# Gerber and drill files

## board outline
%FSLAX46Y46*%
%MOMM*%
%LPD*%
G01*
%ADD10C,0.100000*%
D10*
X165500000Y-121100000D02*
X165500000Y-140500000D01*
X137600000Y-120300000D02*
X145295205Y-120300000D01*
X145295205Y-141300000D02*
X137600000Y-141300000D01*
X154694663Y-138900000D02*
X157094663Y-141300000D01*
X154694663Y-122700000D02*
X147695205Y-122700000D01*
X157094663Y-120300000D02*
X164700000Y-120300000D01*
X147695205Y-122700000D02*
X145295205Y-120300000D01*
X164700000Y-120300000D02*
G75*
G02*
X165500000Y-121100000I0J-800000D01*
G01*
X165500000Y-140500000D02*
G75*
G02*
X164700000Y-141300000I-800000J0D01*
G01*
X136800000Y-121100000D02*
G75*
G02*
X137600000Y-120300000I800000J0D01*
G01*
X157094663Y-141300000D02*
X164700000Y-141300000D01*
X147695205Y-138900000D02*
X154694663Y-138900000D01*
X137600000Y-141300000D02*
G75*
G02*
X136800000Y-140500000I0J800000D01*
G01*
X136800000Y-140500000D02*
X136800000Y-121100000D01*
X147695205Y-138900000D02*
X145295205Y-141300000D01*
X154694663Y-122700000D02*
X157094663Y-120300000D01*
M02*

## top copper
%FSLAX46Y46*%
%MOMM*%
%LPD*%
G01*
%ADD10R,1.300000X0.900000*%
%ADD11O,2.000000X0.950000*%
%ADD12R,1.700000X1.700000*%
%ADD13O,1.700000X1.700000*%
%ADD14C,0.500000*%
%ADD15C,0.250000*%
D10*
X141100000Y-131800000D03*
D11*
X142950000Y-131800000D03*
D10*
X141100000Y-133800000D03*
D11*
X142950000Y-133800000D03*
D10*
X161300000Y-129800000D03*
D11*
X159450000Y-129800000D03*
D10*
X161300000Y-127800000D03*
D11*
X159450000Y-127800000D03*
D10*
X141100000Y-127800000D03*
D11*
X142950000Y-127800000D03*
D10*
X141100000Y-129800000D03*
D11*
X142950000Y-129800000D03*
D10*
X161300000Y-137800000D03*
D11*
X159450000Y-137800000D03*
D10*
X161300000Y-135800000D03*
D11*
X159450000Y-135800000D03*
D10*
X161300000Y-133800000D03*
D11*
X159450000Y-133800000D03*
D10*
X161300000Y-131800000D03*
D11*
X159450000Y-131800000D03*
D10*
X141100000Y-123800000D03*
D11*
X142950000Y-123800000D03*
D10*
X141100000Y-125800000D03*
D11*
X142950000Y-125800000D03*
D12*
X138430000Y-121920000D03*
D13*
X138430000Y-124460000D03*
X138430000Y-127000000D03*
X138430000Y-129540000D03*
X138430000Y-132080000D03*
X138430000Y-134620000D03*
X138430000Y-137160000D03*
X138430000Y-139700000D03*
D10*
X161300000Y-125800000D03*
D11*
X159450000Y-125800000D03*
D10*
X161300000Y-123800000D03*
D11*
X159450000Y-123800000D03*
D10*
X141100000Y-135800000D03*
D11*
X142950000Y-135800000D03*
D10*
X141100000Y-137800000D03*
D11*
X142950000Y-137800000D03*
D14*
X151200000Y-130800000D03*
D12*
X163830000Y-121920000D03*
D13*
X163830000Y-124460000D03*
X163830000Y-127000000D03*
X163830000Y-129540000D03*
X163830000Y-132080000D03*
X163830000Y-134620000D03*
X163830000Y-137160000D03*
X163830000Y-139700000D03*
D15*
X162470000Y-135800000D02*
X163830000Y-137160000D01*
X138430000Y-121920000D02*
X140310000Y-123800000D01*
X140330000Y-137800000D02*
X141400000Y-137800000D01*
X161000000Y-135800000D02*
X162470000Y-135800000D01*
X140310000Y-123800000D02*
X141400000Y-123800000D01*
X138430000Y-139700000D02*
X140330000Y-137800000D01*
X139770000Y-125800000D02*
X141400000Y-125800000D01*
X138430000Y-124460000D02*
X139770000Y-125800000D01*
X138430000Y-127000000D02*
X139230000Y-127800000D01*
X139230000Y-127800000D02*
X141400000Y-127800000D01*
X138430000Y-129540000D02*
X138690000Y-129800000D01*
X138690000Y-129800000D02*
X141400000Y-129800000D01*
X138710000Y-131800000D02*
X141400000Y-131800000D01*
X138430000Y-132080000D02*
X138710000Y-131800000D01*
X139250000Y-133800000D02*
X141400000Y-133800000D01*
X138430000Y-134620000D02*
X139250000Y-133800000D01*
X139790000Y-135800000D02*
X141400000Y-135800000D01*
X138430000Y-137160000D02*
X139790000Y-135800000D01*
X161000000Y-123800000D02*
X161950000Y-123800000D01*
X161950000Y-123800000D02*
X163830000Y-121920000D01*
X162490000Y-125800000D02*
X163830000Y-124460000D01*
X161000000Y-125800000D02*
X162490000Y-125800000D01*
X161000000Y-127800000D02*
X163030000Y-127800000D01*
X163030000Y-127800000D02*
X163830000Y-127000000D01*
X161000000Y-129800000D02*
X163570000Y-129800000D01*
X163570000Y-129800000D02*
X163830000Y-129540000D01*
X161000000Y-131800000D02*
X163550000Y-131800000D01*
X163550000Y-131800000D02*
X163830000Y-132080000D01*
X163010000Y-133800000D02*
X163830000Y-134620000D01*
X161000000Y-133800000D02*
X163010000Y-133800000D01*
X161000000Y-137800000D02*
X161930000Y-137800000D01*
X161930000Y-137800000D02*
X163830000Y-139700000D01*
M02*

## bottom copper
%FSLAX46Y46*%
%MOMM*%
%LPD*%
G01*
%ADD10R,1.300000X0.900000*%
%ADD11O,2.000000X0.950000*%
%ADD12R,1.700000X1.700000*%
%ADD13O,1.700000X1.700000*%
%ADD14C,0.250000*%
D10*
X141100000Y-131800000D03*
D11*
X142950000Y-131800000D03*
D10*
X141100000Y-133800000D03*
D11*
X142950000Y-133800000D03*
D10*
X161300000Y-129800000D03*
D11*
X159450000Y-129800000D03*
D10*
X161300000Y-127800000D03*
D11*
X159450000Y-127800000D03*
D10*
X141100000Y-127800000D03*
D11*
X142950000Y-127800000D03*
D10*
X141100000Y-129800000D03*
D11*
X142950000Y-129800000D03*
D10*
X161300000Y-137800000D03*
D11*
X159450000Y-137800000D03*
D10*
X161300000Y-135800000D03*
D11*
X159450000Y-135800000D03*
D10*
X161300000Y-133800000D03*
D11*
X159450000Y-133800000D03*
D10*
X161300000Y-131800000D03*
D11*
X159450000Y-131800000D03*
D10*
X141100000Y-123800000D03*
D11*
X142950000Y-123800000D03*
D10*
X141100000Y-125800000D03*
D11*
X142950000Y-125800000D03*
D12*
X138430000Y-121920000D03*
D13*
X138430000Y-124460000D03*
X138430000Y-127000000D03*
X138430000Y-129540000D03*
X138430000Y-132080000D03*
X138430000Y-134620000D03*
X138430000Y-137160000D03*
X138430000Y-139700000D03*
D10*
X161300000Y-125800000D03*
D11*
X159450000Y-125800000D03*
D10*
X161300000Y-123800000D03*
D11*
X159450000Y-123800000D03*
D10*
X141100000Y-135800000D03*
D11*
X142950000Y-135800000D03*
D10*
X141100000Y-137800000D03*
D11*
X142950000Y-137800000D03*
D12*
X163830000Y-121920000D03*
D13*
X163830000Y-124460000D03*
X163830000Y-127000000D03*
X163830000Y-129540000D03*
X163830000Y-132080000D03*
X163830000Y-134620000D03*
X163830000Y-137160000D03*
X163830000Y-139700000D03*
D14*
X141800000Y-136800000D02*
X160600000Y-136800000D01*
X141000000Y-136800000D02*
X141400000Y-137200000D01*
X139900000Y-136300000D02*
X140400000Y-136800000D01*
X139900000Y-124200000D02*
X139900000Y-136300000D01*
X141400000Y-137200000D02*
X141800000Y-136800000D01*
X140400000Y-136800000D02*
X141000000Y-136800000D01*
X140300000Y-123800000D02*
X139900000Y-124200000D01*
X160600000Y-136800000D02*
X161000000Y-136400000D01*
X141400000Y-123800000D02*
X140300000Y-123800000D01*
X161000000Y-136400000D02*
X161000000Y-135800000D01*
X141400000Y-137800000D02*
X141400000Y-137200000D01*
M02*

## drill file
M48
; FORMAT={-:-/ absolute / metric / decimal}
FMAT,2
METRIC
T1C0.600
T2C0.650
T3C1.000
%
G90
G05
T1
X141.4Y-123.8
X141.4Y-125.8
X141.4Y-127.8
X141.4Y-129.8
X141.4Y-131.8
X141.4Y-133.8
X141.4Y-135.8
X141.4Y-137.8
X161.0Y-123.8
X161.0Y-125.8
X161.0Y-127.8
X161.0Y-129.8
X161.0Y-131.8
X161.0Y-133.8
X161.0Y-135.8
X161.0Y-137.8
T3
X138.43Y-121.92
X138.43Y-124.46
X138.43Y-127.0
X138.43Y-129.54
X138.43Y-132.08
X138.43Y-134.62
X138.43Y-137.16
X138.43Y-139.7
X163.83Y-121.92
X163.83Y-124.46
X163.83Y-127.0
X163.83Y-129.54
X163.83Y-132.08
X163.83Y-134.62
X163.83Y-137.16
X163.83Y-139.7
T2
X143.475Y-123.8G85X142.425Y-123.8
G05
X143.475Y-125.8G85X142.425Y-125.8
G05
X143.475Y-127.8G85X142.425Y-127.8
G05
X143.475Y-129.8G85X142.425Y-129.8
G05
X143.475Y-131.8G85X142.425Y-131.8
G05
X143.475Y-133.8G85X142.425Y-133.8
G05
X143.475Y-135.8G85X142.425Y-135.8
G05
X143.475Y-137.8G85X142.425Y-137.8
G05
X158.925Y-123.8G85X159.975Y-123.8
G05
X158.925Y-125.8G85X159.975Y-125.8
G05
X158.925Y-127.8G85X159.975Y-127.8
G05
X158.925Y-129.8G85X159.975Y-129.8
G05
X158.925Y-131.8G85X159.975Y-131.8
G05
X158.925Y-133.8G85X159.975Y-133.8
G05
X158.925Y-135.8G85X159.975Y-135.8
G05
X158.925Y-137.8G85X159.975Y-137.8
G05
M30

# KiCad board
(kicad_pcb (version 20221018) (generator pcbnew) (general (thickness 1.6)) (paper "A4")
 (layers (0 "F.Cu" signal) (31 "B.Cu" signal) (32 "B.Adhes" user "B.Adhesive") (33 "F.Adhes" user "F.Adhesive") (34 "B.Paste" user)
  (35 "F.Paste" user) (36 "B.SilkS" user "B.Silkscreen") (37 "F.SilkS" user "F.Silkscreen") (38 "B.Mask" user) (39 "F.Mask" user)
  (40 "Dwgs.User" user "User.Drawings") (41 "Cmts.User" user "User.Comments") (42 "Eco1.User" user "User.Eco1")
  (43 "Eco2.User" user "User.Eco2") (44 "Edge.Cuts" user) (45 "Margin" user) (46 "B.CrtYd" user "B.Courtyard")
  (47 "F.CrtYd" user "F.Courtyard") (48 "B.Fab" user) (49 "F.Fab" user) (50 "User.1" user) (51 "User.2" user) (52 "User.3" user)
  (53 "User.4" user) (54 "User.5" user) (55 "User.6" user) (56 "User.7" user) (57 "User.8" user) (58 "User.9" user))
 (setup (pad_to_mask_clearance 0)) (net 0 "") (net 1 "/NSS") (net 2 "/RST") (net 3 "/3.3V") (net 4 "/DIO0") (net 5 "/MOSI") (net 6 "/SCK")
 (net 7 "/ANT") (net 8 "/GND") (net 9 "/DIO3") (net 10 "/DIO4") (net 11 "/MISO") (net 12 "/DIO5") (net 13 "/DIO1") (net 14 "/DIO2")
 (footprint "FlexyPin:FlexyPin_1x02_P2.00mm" (layer "F.Cu") (at 141.4 131.8)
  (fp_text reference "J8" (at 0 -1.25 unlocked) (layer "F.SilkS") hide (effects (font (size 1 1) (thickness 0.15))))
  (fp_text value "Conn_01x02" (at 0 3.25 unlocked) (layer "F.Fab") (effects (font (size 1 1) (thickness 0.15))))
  (pad "1" thru_hole rect (at 0 0) (size 1.3 0.9) (drill 0.6 (offset -0.3 0)) (layers "*.Cu" "*.Mask") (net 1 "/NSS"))
  (pad "1" thru_hole oval (at 1.55 0 180) (size 2 0.95) (drill oval 1.7 0.65) (layers "*.Cu" "*.Mask") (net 1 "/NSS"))
  (pad "2" thru_hole rect (at 0 2) (size 1.3 0.9) (drill 0.6 (offset -0.3 0)) (layers "*.Cu" "*.Mask") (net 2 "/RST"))
  (pad "2" thru_hole oval (at 1.55 2 180) (size 2 0.95) (drill oval 1.7 0.65) (layers "*.Cu" "*.Mask") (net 2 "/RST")))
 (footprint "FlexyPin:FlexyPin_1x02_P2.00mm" (layer "F.Cu") (at 161 129.8 180)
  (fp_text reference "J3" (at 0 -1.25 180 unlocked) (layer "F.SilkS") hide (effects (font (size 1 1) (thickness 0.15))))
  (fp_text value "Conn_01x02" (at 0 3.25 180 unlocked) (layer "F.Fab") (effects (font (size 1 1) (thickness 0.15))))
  (pad "1" thru_hole rect (at 0 0 180) (size 1.3 0.9) (drill 0.6 (offset -0.3 0)) (layers "*.Cu" "*.Mask") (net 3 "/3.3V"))
  (pad "1" thru_hole oval (at 1.55 0) (size 2 0.95) (drill oval 1.7 0.65) (layers "*.Cu" "*.Mask") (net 3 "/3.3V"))
  (pad "2" thru_hole rect (at 0 2 180) (size 1.3 0.9) (drill 0.6 (offset -0.3 0)) (layers "*.Cu" "*.Mask") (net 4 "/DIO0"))
  (pad "2" thru_hole oval (at 1.55 2) (size 2 0.95) (drill oval 1.7 0.65) (layers "*.Cu" "*.Mask") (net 4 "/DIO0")))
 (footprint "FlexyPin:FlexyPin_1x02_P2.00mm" (layer "F.Cu") (at 141.4 127.8)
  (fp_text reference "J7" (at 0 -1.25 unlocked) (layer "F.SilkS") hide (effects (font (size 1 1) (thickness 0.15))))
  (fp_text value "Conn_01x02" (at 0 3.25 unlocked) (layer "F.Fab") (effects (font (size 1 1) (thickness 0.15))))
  (pad "1" thru_hole rect (at 0 0) (size 1.3 0.9) (drill 0.6 (offset -0.3 0)) (layers "*.Cu" "*.Mask") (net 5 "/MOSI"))
  (pad "1" thru_hole oval (at 1.55 0 180) (size 2 0.95) (drill oval 1.7 0.65) (layers "*.Cu" "*.Mask") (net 5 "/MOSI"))
  (pad "2" thru_hole rect (at 0 2) (size 1.3 0.9) (drill 0.6 (offset -0.3 0)) (layers "*.Cu" "*.Mask") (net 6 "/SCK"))
  (pad "2" thru_hole oval (at 1.55 2 180) (size 2 0.95) (drill oval 1.7 0.65) (layers "*.Cu" "*.Mask") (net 6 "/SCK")))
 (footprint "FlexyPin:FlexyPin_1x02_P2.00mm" (layer "F.Cu") (at 161 137.8 180)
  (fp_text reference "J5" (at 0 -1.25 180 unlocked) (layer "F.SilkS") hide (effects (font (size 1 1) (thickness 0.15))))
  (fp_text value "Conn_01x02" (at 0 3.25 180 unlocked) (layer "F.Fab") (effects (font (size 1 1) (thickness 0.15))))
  (pad "1" thru_hole rect (at 0 0 180) (size 1.3 0.9) (drill 0.6 (offset -0.3 0)) (layers "*.Cu" "*.Mask") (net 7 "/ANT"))
  (pad "1" thru_hole oval (at 1.55 0) (size 2 0.95) (drill oval 1.7 0.65) (layers "*.Cu" "*.Mask") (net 7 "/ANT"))
  (pad "2" thru_hole rect (at 0 2 180) (size 1.3 0.9) (drill 0.6 (offset -0.3 0)) (layers "*.Cu" "*.Mask") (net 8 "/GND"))
  (pad "2" thru_hole oval (at 1.55 2) (size 2 0.95) (drill oval 1.7 0.65) (layers "*.Cu" "*.Mask") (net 8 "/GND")))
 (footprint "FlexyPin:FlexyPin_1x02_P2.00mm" (layer "F.Cu") (at 161 133.8 180)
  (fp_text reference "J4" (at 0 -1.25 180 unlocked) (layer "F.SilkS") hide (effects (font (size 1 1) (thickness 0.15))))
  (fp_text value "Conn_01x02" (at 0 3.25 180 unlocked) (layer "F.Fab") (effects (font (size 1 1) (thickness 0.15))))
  (pad "1" thru_hole rect (at 0 0 180) (size 1.3 0.9) (drill 0.6 (offset -0.3 0)) (layers "*.Cu" "*.Mask") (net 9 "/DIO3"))
  (pad "1" thru_hole oval (at 1.55 0) (size 2 0.95) (drill oval 1.7 0.65) (layers "*.Cu" "*.Mask") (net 9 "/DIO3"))
  (pad "2" thru_hole rect (at 0 2 180) (size 1.3 0.9) (drill 0.6 (offset -0.3 0)) (layers "*.Cu" "*.Mask") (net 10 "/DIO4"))
  (pad "2" thru_hole oval (at 1.55 2) (size 2 0.95) (drill oval 1.7 0.65) (layers "*.Cu" "*.Mask") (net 10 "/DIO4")))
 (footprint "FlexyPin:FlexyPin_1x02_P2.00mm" (layer "F.Cu") (at 141.4 123.8)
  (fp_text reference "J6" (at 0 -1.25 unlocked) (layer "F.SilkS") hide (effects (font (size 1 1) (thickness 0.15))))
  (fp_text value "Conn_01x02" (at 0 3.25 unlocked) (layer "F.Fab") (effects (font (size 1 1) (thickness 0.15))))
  (pad "1" thru_hole rect (at 0 0) (size 1.3 0.9) (drill 0.6 (offset -0.3 0)) (layers "*.Cu" "*.Mask") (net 8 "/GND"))
  (pad "1" thru_hole oval (at 1.55 0 180) (size 2 0.95) (drill oval 1.7 0.65) (layers "*.Cu" "*.Mask") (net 8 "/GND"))
  (pad "2" thru_hole rect (at 0 2) (size 1.3 0.9) (drill 0.6 (offset -0.3 0)) (layers "*.Cu" "*.Mask") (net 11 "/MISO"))
  (pad "2" thru_hole oval (at 1.55 2 180) (size 2 0.95) (drill oval 1.7 0.65) (layers "*.Cu" "*.Mask") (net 11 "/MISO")))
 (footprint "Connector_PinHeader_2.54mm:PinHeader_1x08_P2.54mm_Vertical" (layer "F.Cu") (at 138.43 121.92)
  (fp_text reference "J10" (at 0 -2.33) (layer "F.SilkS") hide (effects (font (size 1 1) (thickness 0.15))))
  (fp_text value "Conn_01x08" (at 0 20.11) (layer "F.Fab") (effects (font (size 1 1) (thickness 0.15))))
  (pad "1" thru_hole rect (at 0 0) (size 1.7 1.7) (drill 1) (layers "*.Cu" "*.Mask") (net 8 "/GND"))
  (pad "2" thru_hole oval (at 0 2.54) (size 1.7 1.7) (drill 1) (layers "*.Cu" "*.Mask") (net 11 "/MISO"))
  (pad "3" thru_hole oval (at 0 5.08) (size 1.7 1.7) (drill 1) (layers "*.Cu" "*.Mask") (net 5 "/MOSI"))
  (pad "4" thru_hole oval (at 0 7.62) (size 1.7 1.7) (drill 1) (layers "*.Cu" "*.Mask") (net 6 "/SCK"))
  (pad "5" thru_hole oval (at 0 10.16) (size 1.7 1.7) (drill 1) (layers "*.Cu" "*.Mask") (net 1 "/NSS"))
  (pad "6" thru_hole oval (at 0 12.7) (size 1.7 1.7) (drill 1) (layers "*.Cu" "*.Mask") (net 2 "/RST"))
  (pad "7" thru_hole oval (at 0 15.24) (size 1.7 1.7) (drill 1) (layers "*.Cu" "*.Mask") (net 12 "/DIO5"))
  (pad "8" thru_hole oval (at 0 17.78) (size 1.7 1.7) (drill 1) (layers "*.Cu" "*.Mask") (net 8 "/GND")))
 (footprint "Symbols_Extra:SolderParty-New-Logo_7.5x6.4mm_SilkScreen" (layer "F.Cu") (at 151.2 135.5)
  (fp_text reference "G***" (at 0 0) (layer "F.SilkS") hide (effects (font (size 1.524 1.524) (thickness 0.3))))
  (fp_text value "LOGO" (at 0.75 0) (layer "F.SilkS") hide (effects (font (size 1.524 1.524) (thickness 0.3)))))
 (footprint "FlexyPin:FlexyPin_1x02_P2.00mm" (layer "F.Cu") (at 161 125.8 180)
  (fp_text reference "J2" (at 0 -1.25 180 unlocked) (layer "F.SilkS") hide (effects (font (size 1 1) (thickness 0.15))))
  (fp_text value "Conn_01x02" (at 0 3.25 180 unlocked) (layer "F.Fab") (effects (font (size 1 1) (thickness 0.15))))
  (pad "1" thru_hole rect (at 0 0 180) (size 1.3 0.9) (drill 0.6 (offset -0.3 0)) (layers "*.Cu" "*.Mask") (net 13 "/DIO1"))
  (pad "1" thru_hole oval (at 1.55 0) (size 2 0.95) (drill oval 1.7 0.65) (layers "*.Cu" "*.Mask") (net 13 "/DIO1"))
  (pad "2" thru_hole rect (at 0 2 180) (size 1.3 0.9) (drill 0.6 (offset -0.3 0)) (layers "*.Cu" "*.Mask") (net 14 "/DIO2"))
  (pad "2" thru_hole oval (at 1.55 2) (size 2 0.95) (drill oval 1.7 0.65) (layers "*.Cu" "*.Mask") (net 14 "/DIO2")))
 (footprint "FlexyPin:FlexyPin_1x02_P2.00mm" (layer "F.Cu") (at 141.4 135.8)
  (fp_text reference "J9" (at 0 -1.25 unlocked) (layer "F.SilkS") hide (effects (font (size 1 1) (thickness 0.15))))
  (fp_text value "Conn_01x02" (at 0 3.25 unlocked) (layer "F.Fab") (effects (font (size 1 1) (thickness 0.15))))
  (pad "1" thru_hole rect (at 0 0) (size 1.3 0.9) (drill 0.6 (offset -0.3 0)) (layers "*.Cu" "*.Mask") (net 12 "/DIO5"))
  (pad "1" thru_hole oval (at 1.55 0 180) (size 2 0.95) (drill oval 1.7 0.65) (layers "*.Cu" "*.Mask") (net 12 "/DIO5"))
  (pad "2" thru_hole rect (at 0 2) (size 1.3 0.9) (drill 0.6 (offset -0.3 0)) (layers "*.Cu" "*.Mask") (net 8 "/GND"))
  (pad "2" thru_hole oval (at 1.55 2 180) (size 2 0.95) (drill oval 1.7 0.65) (layers "*.Cu" "*.Mask") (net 8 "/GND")))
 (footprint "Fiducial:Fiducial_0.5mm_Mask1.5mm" (layer "F.Cu") (at 151.2 130.8)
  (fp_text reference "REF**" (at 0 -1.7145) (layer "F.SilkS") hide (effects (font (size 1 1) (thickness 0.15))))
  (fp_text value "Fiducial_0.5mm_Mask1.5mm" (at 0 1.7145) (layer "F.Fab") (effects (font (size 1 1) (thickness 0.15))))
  (pad "" smd circle (at 0 0) (size 0.5 0.5) (layers "F.Cu") (solder_mask_margin 0.5) (clearance 0.5)))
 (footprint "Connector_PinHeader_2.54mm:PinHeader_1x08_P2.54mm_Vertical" (layer "F.Cu") (at 163.83 121.92)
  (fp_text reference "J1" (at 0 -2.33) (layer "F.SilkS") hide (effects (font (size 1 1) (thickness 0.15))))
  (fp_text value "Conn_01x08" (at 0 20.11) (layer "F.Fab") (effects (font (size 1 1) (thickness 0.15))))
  (pad "1" thru_hole rect (at 0 0) (size 1.7 1.7) (drill 1) (layers "*.Cu" "*.Mask") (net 14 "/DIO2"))
  (pad "2" thru_hole oval (at 0 2.54) (size 1.7 1.7) (drill 1) (layers "*.Cu" "*.Mask") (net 13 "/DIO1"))
  (pad "3" thru_hole oval (at 0 5.08) (size 1.7 1.7) (drill 1) (layers "*.Cu" "*.Mask") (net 4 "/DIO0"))
  (pad "4" thru_hole oval (at 0 7.62) (size 1.7 1.7) (drill 1) (layers "*.Cu" "*.Mask") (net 3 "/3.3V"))
  (pad "5" thru_hole oval (at 0 10.16) (size 1.7 1.7) (drill 1) (layers "*.Cu" "*.Mask") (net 10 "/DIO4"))
  (pad "6" thru_hole oval (at 0 12.7) (size 1.7 1.7) (drill 1) (layers "*.Cu" "*.Mask") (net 9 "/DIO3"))
  (pad "7" thru_hole oval (at 0 15.24) (size 1.7 1.7) (drill 1) (layers "*.Cu" "*.Mask") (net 8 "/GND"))
  (pad "8" thru_hole oval (at 0 17.78) (size 1.7 1.7) (drill 1) (layers "*.Cu" "*.Mask") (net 7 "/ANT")))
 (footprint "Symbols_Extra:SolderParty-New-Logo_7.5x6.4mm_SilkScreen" (layer "B.Cu") (at 150.719476 135 180)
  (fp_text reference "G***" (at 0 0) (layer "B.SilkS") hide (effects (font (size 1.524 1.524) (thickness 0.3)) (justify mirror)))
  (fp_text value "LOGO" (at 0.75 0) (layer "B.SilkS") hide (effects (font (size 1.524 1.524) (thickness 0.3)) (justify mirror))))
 (gr_line (start 165.5 121.1) (end 165.5 140.5) (stroke (width 0.1) (type solid)) (layer "Edge.Cuts"))
 (gr_line (start 137.6 120.3) (end 145.295205 120.3) (stroke (width 0.1) (type solid)) (layer "Edge.Cuts"))
 (gr_line (start 145.295205 141.3) (end 137.6 141.3) (stroke (width 0.1) (type solid)) (layer "Edge.Cuts"))
 (gr_line (start 154.694663 138.9) (end 157.094663 141.3) (stroke (width 0.1) (type solid)) (layer "Edge.Cuts"))
 (gr_line (start 154.694663 122.7) (end 147.695205 122.7) (stroke (width 0.1) (type solid)) (layer "Edge.Cuts"))
 (gr_line (start 157.094663 120.3) (end 164.7 120.3) (stroke (width 0.1) (type solid)) (layer "Edge.Cuts"))
 (gr_line (start 147.695205 122.7) (end 145.295205 120.3) (stroke (width 0.1) (type solid)) (layer "Edge.Cuts"))
 (gr_arc (start 164.7 120.3) (mid 165.265685 120.534315) (end 165.5 121.1) (stroke (width 0.1) (type solid)) (layer "Edge.Cuts"))
 (gr_arc (start 165.5 140.5) (mid 165.265685 141.065685) (end 164.7 141.3) (stroke (width 0.1) (type solid)) (layer "Edge.Cuts"))
 (gr_arc (start 136.8 121.1) (mid 137.034315 120.534315) (end 137.6 120.3) (stroke (width 0.1) (type solid)) (layer "Edge.Cuts"))
 (gr_line (start 157.094663 141.3) (end 164.7 141.3) (stroke (width 0.1) (type solid)) (layer "Edge.Cuts"))
 (gr_line (start 147.695205 138.9) (end 154.694663 138.9) (stroke (width 0.1) (type solid)) (layer "Edge.Cuts"))
 (gr_arc (start 137.6 141.3) (mid 137.034315 141.065685) (end 136.8 140.5) (stroke (width 0.1) (type solid)) (layer "Edge.Cuts"))
 (gr_line (start 136.8 140.5) (end 136.8 121.1) (stroke (width 0.1) (type solid)) (layer "Edge.Cuts"))
 (gr_line (start 147.695205 138.9) (end 145.295205 141.3) (stroke (width 0.1) (type solid)) (layer "Edge.Cuts"))
 (gr_line (start 154.694663 122.7) (end 157.094663 120.3) (stroke (width 0.1) (type solid)) (layer "Edge.Cuts"))
 (segment (start 162.47 135.8) (end 163.83 137.16) (width 0.25) (layer "F.Cu") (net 8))
 (segment (start 138.43 121.92) (end 140.31 123.8) (width 0.25) (layer "F.Cu") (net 8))
 (segment (start 140.33 137.8) (end 141.4 137.8) (width 0.25) (layer "F.Cu") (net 8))
 (segment (start 161 135.8) (end 162.47 135.8) (width 0.25) (layer "F.Cu") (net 8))
 (segment (start 140.31 123.8) (end 141.4 123.8) (width 0.25) (layer "F.Cu") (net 8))
 (segment (start 138.43 139.7) (end 140.33 137.8) (width 0.25) (layer "F.Cu") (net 8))
 (segment (start 141.8 136.8) (end 160.6 136.8) (width 0.25) (layer "B.Cu") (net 8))
 (segment (start 141 136.8) (end 141.4 137.2) (width 0.25) (layer "B.Cu") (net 8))
 (segment (start 139.9 136.3) (end 140.4 136.8) (width 0.25) (layer "B.Cu") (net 8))
 (segment (start 139.9 124.2) (end 139.9 136.3) (width 0.25) (layer "B.Cu") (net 8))
 (segment (start 141.4 137.2) (end 141.8 136.8) (width 0.25) (layer "B.Cu") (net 8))
 (segment (start 140.4 136.8) (end 141 136.8) (width 0.25) (layer "B.Cu") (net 8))
 (segment (start 140.3 123.8) (end 139.9 124.2) (width 0.25) (layer "B.Cu") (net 8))
 (segment (start 160.6 136.8) (end 161 136.4) (width 0.25) (layer "B.Cu") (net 8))
 (segment (start 141.4 123.8) (end 140.3 123.8) (width 0.25) (layer "B.Cu") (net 8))
 (segment (start 161 136.4) (end 161 135.8) (width 0.25) (layer "B.Cu") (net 8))
 (segment (start 141.4 137.8) (end 141.4 137.2) (width 0.25) (layer "B.Cu") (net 8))
 (segment (start 139.77 125.8) (end 141.4 125.8) (width 0.25) (layer "F.Cu") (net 11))
 (segment (start 138.43 124.46) (end 139.77 125.8) (width 0.25) (layer "F.Cu") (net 11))
 (segment (start 138.43 127) (end 139.23 127.8) (width 0.25) (layer "F.Cu") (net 5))
 (segment (start 139.23 127.8) (end 141.4 127.8) (width 0.25) (layer "F.Cu") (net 5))
 (segment (start 138.43 129.54) (end 138.69 129.8) (width 0.25) (layer "F.Cu") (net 6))
 (segment (start 138.69 129.8) (end 141.4 129.8) (width 0.25) (layer "F.Cu") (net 6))
 (segment (start 138.71 131.8) (end 141.4 131.8) (width 0.25) (layer "F.Cu") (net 1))
 (segment (start 138.43 132.08) (end 138.71 131.8) (width 0.25) (layer "F.Cu") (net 1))
 (segment (start 139.25 133.8) (end 141.4 133.8) (width 0.25) (layer "F.Cu") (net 2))
 (segment (start 138.43 134.62) (end 139.25 133.8) (width 0.25) (layer "F.Cu") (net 2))
 (segment (start 139.79 135.8) (end 141.4 135.8) (width 0.25) (layer "F.Cu") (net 12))
 (segment (start 138.43 137.16) (end 139.79 135.8) (width 0.25) (layer "F.Cu") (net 12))
 (segment (start 161 123.8) (end 161.95 123.8) (width 0.25) (layer "F.Cu") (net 14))
 (segment (start 161.95 123.8) (end 163.83 121.92) (width 0.25) (layer "F.Cu") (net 14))
 (segment (start 162.49 125.8) (end 163.83 124.46) (width 0.25) (layer "F.Cu") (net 13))
 (segment (start 161 125.8) (end 162.49 125.8) (width 0.25) (layer "F.Cu") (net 13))
 (segment (start 161 127.8) (end 163.03 127.8) (width 0.25) (layer "F.Cu") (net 4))
 (segment (start 163.03 127.8) (end 163.83 127) (width 0.25) (layer "F.Cu") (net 4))
 (segment (start 161 129.8) (end 163.57 129.8) (width 0.25) (layer "F.Cu") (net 3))
 (segment (start 163.57 129.8) (end 163.83 129.54) (width 0.25) (layer "F.Cu") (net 3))
 (segment (start 161 131.8) (end 163.55 131.8) (width 0.25) (layer "F.Cu") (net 10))
 (segment (start 163.55 131.8) (end 163.83 132.08) (width 0.25) (layer "F.Cu") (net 10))
 (segment (start 163.01 133.8) (end 163.83 134.62) (width 0.25) (layer "F.Cu") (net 9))
 (segment (start 161 133.8) (end 163.01 133.8) (width 0.25) (layer "F.Cu") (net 9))
 (segment (start 161 137.8) (end 161.93 137.8) (width 0.25) (layer "F.Cu") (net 7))
 (segment (start 161.93 137.8) (end 163.83 139.7) (width 0.25) (layer "F.Cu") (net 7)))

